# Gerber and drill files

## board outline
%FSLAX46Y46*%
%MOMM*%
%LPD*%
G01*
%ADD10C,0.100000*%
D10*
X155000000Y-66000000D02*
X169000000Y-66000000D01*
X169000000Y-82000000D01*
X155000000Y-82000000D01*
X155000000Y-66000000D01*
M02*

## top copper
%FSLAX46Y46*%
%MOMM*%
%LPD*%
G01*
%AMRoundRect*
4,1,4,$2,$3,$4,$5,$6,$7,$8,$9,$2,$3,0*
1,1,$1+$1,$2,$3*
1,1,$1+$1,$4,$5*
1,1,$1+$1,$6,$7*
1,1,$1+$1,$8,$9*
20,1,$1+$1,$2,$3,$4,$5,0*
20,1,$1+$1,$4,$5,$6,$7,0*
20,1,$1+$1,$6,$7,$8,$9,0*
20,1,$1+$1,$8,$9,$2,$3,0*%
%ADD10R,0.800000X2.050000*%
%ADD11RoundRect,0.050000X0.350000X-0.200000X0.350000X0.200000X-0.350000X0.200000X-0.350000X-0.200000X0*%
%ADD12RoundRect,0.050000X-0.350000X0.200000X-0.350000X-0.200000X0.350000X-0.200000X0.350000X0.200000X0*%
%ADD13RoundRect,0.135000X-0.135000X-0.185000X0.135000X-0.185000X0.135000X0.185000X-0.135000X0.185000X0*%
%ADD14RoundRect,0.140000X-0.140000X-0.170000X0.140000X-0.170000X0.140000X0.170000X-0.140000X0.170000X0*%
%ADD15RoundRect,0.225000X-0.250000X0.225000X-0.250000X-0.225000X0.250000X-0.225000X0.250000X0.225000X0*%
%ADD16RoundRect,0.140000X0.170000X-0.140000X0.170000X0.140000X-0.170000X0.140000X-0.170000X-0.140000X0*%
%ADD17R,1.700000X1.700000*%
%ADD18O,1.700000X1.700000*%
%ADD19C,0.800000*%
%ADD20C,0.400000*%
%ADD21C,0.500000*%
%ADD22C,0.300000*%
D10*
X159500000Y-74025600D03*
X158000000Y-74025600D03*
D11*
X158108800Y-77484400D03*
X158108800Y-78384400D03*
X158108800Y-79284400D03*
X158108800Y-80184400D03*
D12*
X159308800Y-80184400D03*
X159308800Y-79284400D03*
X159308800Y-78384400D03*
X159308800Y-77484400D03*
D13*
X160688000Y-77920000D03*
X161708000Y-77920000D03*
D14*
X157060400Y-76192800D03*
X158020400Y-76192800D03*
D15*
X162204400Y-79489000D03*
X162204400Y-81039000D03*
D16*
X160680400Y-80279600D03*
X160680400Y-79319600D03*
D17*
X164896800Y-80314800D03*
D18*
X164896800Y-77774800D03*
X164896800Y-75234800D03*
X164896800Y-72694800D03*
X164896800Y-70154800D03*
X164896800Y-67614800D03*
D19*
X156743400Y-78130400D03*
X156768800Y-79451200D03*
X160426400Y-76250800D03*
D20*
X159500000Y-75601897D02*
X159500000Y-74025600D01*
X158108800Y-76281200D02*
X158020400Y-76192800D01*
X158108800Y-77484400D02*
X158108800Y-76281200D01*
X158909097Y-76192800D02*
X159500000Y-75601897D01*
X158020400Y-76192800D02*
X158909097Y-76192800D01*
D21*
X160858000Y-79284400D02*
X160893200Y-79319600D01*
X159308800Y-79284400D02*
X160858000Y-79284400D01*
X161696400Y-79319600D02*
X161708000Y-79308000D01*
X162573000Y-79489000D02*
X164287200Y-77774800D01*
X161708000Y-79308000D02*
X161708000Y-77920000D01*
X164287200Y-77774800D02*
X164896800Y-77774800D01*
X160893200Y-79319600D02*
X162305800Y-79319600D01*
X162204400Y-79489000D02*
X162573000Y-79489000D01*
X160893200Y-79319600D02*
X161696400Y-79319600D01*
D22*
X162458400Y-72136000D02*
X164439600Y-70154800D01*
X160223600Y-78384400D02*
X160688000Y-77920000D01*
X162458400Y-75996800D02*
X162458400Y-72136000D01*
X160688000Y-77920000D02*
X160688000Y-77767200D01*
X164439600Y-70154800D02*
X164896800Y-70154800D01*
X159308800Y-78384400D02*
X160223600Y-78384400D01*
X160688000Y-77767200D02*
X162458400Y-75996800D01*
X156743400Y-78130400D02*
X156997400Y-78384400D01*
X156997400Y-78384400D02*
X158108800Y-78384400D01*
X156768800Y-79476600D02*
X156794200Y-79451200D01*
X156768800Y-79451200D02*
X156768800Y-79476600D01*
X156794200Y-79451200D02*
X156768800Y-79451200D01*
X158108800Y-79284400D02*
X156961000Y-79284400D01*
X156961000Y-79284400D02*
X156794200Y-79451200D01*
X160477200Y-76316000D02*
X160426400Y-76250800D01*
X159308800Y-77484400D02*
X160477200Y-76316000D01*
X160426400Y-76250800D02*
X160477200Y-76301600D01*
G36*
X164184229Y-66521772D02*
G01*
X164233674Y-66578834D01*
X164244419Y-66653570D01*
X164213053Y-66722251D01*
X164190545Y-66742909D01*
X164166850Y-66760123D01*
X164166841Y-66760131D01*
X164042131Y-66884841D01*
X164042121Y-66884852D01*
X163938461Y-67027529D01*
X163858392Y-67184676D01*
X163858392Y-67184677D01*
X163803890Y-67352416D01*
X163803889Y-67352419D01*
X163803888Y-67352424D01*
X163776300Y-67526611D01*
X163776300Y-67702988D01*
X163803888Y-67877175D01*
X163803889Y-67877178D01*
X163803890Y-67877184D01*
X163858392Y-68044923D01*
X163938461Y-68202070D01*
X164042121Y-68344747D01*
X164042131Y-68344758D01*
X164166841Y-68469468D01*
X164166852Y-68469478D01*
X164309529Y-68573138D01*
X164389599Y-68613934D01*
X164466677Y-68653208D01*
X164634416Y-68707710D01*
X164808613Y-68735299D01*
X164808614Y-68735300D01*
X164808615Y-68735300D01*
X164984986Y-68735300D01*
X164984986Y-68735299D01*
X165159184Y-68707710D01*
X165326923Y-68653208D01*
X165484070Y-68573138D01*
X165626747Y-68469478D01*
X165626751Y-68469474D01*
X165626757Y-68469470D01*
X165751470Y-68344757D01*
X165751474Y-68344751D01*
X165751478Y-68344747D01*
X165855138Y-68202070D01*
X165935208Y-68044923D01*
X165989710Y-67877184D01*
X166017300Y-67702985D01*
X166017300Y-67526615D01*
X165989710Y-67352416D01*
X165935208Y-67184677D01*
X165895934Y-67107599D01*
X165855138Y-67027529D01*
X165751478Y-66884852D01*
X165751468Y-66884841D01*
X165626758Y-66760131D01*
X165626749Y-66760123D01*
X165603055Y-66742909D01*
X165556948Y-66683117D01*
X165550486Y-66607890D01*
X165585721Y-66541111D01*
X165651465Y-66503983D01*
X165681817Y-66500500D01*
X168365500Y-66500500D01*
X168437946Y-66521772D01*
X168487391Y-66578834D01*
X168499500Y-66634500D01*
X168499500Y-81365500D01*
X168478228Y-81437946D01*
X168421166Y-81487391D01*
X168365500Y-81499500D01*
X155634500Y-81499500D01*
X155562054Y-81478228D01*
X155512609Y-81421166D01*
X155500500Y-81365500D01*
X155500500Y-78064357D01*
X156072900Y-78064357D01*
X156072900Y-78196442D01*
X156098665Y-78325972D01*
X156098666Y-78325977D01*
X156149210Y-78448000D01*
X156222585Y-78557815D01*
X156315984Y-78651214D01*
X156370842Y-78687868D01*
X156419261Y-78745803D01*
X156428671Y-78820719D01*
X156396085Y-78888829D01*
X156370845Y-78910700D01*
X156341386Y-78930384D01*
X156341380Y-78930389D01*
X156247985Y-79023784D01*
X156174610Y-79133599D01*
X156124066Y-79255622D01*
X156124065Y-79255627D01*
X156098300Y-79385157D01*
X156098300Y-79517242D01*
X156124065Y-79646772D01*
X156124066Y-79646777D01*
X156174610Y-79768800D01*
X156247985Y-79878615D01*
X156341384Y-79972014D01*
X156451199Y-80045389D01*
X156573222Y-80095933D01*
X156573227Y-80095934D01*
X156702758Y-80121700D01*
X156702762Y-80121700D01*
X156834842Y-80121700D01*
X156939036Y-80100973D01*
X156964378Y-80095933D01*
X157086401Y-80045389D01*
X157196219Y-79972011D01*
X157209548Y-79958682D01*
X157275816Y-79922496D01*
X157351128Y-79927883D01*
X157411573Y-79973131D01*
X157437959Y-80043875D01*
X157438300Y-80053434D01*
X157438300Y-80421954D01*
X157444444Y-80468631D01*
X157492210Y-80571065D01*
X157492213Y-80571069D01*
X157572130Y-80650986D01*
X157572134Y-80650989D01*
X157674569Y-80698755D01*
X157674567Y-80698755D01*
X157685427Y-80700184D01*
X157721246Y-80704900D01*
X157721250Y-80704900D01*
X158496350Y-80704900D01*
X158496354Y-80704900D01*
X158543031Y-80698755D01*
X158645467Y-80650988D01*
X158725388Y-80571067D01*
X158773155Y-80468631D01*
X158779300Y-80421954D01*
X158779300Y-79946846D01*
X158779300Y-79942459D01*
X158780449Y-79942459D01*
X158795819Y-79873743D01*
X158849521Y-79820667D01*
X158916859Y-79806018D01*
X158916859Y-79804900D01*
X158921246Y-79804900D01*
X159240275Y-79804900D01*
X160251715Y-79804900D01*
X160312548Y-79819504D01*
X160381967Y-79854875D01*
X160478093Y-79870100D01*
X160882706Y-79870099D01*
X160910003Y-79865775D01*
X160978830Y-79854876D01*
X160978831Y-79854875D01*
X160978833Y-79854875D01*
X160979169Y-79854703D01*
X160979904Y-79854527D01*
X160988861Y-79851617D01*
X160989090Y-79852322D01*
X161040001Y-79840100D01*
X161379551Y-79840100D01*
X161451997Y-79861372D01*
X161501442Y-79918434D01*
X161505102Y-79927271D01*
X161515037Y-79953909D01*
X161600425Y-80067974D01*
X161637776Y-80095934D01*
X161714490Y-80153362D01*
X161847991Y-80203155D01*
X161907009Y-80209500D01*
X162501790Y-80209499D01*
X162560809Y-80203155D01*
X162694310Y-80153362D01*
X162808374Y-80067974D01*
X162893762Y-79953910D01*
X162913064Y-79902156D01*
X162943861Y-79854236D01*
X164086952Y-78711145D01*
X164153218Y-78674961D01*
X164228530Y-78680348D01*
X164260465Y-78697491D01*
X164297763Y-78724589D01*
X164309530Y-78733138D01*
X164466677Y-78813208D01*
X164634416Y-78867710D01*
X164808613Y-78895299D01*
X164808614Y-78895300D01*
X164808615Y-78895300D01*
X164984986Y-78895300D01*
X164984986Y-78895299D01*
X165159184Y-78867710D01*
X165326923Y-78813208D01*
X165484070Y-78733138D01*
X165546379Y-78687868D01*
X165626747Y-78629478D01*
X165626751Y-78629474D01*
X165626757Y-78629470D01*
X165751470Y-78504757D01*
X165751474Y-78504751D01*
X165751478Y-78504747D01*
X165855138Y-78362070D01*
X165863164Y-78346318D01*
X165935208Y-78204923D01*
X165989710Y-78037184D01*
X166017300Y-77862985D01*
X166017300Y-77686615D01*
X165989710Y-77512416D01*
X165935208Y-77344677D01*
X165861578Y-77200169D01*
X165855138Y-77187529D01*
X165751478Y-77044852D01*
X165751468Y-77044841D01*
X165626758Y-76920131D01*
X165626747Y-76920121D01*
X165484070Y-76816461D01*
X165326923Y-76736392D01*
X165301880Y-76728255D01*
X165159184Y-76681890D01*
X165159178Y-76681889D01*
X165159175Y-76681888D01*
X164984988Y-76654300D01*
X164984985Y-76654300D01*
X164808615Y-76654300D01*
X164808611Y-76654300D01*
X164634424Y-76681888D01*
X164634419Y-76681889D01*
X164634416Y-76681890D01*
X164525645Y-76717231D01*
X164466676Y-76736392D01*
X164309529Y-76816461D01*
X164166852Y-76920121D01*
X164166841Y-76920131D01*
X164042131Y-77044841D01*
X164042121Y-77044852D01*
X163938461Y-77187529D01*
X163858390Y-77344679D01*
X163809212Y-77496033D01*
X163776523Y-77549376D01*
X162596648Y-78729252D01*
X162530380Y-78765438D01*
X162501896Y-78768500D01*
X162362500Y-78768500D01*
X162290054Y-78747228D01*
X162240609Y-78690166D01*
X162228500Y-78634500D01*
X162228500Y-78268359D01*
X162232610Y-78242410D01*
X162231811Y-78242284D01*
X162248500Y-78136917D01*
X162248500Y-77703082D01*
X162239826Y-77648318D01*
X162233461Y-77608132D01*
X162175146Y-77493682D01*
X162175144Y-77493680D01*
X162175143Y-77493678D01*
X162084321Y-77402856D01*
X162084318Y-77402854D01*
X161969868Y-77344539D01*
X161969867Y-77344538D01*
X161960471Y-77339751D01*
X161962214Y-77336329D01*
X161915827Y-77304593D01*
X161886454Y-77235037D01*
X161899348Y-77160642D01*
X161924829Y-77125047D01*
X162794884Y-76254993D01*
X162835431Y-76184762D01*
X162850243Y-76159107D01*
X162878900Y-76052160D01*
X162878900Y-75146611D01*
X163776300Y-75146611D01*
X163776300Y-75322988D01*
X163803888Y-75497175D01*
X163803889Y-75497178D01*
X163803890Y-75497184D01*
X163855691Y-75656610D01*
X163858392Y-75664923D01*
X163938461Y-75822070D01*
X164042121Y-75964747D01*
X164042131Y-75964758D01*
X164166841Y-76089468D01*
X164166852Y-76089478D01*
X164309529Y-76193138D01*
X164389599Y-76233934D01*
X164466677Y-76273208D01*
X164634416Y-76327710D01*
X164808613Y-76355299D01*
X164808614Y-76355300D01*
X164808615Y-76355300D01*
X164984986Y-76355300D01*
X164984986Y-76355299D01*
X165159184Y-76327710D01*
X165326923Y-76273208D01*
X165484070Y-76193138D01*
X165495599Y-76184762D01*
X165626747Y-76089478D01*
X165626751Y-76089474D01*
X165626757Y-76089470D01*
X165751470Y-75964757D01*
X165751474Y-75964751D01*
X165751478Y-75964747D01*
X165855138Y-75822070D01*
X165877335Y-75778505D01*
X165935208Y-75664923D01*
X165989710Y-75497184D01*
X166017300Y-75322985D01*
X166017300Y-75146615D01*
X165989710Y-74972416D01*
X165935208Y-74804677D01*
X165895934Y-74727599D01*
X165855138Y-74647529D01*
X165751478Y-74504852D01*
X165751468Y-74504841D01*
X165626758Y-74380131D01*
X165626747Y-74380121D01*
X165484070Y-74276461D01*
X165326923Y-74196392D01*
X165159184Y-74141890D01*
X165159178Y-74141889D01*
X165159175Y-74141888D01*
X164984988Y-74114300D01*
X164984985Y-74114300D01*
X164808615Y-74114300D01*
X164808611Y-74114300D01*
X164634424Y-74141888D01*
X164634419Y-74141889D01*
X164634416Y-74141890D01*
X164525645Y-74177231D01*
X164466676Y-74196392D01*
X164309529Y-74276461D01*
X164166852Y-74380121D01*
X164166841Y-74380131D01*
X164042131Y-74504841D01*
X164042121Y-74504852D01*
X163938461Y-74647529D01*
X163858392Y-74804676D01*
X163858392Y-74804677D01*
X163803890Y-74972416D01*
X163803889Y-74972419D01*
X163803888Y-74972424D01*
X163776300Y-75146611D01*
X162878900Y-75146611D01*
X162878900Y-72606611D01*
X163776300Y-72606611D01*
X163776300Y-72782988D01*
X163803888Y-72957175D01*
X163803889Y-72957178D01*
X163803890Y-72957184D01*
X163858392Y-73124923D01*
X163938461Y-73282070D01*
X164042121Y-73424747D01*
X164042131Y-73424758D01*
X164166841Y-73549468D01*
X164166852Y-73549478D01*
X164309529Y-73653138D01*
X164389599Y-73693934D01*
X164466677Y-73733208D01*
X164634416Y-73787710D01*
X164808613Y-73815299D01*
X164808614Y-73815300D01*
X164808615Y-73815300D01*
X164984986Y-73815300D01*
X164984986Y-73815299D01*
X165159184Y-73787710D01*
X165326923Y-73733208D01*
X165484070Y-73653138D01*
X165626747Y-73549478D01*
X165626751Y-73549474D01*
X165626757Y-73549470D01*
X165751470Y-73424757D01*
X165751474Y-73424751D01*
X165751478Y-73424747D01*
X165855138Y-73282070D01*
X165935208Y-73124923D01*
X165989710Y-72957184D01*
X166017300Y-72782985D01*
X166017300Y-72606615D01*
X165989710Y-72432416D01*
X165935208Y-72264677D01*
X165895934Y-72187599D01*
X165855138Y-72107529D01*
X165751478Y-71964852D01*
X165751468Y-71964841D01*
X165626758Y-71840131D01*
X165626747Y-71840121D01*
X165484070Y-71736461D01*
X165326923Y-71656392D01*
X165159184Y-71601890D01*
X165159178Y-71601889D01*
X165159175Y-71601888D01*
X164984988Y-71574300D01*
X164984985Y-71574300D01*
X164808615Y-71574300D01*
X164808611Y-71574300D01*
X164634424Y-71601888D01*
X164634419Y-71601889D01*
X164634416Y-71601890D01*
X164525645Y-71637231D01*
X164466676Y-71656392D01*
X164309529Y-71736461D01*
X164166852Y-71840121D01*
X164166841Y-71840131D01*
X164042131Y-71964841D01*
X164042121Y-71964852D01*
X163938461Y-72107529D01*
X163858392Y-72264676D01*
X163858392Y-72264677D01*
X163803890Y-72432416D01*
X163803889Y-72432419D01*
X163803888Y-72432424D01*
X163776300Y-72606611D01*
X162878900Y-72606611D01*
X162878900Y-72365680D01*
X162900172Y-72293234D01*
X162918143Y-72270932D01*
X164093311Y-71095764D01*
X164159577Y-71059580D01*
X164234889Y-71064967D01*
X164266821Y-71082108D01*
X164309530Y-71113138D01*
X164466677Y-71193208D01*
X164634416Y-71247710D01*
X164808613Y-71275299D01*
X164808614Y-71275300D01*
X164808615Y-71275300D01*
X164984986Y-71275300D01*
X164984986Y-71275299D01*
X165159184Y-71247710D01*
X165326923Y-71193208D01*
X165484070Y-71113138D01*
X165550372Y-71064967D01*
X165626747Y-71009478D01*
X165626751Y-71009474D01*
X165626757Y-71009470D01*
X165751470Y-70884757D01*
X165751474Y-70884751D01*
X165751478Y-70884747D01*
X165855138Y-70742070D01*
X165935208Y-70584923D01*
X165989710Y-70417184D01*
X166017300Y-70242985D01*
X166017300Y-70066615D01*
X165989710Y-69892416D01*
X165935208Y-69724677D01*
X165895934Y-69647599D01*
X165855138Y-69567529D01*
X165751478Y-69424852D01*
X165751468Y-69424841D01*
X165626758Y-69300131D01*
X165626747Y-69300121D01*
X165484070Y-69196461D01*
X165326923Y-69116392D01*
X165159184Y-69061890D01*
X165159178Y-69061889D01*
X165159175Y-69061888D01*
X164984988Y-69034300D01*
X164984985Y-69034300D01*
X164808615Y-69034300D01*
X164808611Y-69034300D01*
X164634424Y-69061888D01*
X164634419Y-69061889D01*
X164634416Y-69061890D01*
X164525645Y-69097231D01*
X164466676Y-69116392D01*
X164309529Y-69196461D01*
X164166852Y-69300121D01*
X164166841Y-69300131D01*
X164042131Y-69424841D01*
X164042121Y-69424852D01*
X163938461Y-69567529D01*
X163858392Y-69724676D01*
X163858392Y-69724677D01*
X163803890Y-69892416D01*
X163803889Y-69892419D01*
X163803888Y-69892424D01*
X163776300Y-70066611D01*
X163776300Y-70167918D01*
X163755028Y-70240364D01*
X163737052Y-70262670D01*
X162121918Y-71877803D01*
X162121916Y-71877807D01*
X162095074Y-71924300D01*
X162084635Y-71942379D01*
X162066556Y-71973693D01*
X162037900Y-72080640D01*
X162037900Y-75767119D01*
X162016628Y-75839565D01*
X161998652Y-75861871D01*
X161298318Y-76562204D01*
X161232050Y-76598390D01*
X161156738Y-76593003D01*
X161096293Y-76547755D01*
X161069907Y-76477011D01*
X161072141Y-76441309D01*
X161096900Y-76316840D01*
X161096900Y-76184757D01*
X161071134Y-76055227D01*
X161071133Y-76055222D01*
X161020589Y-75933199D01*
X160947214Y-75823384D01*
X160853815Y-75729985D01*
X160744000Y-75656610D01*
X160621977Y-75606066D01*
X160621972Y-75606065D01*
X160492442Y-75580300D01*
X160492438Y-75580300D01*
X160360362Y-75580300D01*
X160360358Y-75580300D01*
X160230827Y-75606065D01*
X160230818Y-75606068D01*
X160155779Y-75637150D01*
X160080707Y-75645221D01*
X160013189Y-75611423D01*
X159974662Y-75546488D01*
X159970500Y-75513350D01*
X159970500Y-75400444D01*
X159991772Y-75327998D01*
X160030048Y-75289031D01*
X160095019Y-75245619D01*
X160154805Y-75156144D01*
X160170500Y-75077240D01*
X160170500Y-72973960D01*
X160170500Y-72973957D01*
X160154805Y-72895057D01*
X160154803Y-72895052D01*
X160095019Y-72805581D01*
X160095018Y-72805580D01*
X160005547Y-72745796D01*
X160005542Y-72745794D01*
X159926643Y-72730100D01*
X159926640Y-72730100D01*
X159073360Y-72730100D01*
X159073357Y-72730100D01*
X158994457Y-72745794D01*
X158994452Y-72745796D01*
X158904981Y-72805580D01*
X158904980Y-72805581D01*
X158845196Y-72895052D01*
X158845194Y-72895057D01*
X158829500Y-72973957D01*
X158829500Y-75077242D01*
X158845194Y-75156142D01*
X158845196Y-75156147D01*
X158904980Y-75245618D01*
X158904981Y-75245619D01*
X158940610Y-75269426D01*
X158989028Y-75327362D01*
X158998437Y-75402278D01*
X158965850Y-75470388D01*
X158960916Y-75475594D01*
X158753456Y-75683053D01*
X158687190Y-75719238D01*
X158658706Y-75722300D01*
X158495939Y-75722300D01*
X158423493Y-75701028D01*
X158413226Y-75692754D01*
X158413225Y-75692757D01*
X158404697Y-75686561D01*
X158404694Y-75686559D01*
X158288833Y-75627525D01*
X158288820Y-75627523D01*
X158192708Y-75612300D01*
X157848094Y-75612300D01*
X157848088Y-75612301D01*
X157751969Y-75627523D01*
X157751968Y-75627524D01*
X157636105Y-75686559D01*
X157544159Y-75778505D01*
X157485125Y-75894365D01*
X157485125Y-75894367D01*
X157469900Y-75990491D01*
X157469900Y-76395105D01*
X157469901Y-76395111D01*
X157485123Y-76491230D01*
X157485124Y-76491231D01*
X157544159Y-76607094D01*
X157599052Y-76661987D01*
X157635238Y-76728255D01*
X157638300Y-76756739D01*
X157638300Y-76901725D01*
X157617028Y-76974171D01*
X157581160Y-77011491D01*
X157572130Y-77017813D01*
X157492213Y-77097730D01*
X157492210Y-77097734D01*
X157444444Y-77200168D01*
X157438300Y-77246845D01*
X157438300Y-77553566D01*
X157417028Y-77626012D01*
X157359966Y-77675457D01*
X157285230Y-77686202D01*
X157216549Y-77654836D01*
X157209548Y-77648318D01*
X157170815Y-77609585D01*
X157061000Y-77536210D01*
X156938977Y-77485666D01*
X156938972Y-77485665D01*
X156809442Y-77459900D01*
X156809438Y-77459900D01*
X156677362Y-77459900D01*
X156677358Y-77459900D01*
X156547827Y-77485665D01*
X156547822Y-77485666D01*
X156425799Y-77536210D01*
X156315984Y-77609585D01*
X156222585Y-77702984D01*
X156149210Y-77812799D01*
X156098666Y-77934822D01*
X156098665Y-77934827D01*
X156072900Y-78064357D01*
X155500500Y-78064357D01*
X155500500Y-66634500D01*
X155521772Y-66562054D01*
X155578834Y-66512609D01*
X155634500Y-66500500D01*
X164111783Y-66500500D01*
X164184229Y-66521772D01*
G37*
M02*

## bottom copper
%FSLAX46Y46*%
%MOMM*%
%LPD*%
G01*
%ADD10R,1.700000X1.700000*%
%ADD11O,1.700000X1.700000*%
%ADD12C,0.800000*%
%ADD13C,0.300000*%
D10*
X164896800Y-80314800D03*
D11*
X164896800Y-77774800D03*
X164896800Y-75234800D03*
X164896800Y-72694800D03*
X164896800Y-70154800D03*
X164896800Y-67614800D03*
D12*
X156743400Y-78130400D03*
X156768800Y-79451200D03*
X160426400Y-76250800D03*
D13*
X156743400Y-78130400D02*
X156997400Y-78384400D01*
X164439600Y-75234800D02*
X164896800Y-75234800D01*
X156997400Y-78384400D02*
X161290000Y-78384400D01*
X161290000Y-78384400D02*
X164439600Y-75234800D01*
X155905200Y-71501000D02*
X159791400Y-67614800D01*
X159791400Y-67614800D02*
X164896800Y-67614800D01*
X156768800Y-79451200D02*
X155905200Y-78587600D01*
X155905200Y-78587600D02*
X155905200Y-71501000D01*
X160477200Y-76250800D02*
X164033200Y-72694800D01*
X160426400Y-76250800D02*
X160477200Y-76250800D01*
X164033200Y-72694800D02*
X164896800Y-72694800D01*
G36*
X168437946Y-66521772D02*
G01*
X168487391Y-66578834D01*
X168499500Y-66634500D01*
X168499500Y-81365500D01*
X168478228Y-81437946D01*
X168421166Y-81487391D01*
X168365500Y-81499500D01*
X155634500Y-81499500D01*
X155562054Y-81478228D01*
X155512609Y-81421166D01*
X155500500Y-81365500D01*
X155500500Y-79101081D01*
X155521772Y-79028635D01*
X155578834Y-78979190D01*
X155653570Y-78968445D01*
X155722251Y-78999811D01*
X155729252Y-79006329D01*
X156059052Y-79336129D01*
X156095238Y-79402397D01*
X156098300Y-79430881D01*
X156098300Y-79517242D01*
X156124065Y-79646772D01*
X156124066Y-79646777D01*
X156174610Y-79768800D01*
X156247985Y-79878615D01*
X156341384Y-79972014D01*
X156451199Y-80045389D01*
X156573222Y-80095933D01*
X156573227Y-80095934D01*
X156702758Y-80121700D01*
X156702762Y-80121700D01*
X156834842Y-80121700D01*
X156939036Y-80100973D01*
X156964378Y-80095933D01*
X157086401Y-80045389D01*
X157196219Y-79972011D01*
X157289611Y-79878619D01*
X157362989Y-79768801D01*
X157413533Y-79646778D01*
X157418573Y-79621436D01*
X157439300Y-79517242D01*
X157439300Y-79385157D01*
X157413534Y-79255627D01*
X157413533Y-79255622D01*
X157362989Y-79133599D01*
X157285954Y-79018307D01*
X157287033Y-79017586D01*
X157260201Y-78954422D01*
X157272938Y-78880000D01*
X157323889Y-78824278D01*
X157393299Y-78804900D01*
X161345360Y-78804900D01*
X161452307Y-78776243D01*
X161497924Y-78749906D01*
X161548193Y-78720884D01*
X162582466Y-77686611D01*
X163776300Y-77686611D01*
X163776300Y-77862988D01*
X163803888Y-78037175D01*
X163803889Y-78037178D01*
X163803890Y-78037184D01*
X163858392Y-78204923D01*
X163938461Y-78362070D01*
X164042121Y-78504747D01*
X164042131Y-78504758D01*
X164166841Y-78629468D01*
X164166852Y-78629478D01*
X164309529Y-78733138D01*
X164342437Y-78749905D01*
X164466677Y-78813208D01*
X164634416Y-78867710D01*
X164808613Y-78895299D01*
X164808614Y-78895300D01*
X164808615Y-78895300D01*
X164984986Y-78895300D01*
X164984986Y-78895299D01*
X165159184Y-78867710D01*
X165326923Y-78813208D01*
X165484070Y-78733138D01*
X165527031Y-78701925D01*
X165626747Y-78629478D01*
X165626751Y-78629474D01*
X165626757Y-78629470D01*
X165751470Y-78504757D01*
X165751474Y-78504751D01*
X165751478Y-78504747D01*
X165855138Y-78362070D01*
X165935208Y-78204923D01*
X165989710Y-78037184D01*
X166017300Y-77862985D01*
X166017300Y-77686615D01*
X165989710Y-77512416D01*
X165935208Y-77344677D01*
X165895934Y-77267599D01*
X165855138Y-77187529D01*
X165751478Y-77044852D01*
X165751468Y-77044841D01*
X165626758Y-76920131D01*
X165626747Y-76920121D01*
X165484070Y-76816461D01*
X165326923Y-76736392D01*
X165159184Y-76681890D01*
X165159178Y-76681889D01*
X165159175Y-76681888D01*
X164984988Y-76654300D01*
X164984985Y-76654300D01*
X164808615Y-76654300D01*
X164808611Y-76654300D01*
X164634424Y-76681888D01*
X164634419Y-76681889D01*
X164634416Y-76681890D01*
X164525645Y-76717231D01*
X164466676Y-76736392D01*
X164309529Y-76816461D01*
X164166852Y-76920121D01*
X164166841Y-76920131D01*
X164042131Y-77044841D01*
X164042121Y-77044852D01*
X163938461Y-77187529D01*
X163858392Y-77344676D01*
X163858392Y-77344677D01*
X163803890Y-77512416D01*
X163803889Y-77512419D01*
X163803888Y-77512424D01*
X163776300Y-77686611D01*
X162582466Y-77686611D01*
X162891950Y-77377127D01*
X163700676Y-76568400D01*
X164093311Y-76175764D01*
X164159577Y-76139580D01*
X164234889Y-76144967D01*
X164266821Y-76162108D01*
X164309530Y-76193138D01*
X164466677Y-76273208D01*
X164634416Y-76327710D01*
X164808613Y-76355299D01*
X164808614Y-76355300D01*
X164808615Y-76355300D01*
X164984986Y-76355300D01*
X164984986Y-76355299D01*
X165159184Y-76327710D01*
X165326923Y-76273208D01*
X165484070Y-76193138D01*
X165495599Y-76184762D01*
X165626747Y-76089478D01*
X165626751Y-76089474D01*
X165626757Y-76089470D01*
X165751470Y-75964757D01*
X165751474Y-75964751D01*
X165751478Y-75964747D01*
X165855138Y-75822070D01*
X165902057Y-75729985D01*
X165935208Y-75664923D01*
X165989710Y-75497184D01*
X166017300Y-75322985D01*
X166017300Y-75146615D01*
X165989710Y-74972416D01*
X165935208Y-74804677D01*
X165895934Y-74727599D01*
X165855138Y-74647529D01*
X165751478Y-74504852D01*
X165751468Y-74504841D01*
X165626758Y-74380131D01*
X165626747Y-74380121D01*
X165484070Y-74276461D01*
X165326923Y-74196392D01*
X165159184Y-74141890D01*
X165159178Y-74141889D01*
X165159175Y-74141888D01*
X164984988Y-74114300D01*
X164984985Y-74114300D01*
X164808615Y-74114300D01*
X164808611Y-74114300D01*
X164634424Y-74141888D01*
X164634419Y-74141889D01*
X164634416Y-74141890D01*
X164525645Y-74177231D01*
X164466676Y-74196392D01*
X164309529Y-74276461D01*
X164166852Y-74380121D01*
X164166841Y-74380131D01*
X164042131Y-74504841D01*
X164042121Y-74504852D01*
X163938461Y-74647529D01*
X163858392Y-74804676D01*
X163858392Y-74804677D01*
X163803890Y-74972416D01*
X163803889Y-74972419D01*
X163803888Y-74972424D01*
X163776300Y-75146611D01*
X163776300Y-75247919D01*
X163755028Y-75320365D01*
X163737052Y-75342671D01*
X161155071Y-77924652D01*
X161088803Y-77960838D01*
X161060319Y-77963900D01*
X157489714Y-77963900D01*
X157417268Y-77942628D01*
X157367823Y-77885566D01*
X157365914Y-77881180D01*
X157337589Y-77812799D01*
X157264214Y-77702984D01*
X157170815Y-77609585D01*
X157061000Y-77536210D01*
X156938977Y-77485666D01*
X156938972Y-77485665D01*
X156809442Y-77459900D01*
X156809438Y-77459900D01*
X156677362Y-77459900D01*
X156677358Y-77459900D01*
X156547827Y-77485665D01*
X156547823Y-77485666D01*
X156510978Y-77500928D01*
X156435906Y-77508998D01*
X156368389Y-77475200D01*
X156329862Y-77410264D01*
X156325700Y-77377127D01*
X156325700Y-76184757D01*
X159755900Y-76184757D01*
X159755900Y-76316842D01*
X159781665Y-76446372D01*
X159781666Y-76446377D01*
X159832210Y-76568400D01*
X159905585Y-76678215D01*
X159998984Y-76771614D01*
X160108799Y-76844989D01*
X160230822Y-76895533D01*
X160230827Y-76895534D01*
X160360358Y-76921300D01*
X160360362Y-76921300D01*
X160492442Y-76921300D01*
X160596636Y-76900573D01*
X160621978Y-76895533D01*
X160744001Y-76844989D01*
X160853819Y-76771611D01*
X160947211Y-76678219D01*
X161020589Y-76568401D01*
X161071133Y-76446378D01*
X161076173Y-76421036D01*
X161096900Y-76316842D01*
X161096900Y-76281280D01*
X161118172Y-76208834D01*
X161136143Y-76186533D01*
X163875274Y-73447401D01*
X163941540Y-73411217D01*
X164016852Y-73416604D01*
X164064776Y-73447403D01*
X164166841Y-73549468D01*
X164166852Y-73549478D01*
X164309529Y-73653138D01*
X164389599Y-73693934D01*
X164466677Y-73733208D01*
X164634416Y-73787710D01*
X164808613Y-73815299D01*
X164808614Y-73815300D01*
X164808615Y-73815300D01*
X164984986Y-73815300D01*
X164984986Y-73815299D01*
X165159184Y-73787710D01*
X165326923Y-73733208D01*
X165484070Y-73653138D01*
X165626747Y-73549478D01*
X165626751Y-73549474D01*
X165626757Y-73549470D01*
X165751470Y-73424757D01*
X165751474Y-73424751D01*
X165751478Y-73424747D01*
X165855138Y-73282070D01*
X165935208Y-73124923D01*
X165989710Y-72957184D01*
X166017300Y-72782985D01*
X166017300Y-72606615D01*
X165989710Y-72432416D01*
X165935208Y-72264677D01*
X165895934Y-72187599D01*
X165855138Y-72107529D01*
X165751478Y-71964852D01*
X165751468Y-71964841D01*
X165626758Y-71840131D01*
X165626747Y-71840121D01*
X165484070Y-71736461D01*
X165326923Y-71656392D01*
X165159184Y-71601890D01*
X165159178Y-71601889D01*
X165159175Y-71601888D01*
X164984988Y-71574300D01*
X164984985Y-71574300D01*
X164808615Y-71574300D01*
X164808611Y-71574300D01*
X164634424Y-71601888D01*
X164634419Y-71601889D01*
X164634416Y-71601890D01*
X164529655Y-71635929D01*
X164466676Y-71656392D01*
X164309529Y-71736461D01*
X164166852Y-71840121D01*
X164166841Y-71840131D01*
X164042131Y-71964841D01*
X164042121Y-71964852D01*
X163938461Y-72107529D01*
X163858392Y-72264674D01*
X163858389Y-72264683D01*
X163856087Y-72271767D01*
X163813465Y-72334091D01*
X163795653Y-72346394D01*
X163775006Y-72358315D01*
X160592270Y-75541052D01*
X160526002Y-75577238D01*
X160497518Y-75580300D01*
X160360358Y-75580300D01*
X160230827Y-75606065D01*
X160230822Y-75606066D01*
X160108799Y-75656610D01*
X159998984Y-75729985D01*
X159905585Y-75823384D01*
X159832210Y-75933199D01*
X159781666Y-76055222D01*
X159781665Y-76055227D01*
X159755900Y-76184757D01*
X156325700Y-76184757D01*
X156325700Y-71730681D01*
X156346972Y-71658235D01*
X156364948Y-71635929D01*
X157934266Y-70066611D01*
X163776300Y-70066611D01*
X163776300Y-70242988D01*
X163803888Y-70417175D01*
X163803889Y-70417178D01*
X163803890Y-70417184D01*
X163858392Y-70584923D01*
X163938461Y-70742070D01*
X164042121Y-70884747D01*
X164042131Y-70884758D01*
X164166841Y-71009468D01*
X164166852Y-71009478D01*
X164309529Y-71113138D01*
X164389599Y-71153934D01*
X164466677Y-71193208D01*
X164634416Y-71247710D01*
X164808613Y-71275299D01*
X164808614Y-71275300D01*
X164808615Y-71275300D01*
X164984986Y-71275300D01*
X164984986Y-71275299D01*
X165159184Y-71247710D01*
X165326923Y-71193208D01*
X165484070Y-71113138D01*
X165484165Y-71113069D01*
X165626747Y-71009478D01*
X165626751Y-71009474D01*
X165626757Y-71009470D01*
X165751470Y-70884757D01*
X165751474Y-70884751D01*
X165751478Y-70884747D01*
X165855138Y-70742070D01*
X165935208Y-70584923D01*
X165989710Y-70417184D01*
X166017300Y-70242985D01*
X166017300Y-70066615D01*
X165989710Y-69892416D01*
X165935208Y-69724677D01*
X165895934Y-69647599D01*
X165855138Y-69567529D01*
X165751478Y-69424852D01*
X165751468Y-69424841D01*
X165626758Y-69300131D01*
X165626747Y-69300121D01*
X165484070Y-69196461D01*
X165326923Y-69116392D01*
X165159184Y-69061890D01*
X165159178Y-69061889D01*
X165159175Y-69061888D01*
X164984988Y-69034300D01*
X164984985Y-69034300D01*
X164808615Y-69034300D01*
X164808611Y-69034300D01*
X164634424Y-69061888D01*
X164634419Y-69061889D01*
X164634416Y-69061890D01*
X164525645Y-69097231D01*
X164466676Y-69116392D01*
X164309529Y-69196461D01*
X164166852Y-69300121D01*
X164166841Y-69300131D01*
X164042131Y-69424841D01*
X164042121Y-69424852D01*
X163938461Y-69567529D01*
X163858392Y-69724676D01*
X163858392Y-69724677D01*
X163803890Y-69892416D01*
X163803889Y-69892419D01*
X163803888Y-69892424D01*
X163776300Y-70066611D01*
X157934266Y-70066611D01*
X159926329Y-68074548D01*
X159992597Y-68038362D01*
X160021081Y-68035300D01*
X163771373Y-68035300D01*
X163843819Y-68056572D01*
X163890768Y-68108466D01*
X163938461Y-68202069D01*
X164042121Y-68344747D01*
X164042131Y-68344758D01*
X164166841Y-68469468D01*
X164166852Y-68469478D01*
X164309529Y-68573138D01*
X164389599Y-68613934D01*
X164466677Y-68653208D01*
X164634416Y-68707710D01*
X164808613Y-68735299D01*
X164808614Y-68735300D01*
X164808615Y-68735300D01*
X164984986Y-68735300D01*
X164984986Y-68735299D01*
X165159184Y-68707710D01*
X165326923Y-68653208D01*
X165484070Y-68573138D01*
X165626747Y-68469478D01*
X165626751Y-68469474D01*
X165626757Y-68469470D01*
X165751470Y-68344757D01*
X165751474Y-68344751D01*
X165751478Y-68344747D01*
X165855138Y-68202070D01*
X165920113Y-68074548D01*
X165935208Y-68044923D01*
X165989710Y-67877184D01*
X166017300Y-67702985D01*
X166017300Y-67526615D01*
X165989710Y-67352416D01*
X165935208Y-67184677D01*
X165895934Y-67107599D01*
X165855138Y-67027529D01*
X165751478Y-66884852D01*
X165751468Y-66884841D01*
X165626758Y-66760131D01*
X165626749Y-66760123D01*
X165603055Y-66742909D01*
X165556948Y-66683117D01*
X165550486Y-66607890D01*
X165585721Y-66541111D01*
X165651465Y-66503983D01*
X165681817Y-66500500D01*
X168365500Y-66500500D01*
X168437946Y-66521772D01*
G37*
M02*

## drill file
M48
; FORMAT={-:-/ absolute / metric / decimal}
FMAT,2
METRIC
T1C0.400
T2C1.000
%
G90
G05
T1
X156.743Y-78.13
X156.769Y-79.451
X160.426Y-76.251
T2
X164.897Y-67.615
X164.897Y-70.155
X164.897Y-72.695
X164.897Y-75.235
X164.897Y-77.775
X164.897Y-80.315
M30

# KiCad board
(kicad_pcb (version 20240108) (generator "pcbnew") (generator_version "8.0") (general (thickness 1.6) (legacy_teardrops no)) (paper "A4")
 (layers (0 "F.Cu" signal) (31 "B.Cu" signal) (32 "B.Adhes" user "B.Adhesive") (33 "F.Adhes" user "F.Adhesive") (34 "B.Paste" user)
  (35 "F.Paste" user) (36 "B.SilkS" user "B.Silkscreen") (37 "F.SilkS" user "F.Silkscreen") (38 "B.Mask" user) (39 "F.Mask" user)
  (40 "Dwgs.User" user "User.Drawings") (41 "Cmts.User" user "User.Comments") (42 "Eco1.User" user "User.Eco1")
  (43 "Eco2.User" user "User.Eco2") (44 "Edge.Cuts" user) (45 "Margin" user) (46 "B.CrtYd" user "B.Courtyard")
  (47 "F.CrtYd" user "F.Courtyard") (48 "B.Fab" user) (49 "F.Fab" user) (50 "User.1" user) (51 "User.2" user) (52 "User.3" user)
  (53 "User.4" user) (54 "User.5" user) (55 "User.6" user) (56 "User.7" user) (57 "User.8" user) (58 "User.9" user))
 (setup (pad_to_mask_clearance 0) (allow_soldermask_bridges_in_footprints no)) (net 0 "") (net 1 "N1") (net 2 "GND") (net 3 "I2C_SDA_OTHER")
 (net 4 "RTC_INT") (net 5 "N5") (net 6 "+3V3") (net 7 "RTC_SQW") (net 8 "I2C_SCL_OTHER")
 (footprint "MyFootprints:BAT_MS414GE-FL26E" (layer "F.Cu") (at 158.75 70.3006 -90)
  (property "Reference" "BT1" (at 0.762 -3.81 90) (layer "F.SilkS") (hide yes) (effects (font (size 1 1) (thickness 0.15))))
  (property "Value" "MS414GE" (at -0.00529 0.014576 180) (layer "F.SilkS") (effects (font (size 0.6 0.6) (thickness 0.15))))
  (pad "1" smd rect (at 3.725 -0.75 270) (size 2.05 0.8) (layers "F.Cu" "F.Paste" "F.Mask") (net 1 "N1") (solder_mask_margin 0.102))
  (pad "2" smd rect (at 3.725 0.75 270) (size 2.05 0.8) (layers "F.Cu" "F.Paste" "F.Mask") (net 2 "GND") (solder_mask_margin 0.102)))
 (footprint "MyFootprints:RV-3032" (layer "F.Cu") (at 158.7088 78.8344 -90)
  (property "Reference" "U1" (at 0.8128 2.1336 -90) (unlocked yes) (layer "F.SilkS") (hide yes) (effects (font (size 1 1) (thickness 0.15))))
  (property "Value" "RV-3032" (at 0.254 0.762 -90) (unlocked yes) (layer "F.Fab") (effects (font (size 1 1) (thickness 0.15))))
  (pad "1" smd roundrect (at -1.35 0.6 90) (size 0.5 0.8) (layers "F.Cu" "F.Paste" "F.Mask") (roundrect_rratio 0.1) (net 1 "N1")
   (thermal_bridge_angle 45))
  (pad "2" smd roundrect (at -0.45 0.6 90) (size 0.5 0.8) (layers "F.Cu" "F.Paste" "F.Mask") (roundrect_rratio 0.1) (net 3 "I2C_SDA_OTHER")
   (thermal_bridge_angle 45))
  (pad "3" smd roundrect (at 0.45 0.6 90) (size 0.5 0.8) (layers "F.Cu" "F.Paste" "F.Mask") (roundrect_rratio 0.1) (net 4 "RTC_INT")
   (thermal_bridge_angle 45))
  (pad "4" smd roundrect (at 1.35 0.6 90) (size 0.5 0.8) (layers "F.Cu" "F.Paste" "F.Mask") (roundrect_rratio 0.1) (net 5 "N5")
   (thermal_bridge_angle 45))
  (pad "5" smd roundrect (at 1.35 -0.6 270) (size 0.5 0.8) (layers "F.Cu" "F.Paste" "F.Mask") (roundrect_rratio 0.1) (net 2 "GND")
   (thermal_bridge_angle 45))
  (pad "6" smd roundrect (at 0.45 -0.6 270) (size 0.5 0.8) (layers "F.Cu" "F.Paste" "F.Mask") (roundrect_rratio 0.1) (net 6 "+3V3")
   (thermal_bridge_angle 45))
  (pad "7" smd roundrect (at -0.45 -0.6 270) (size 0.5 0.8) (layers "F.Cu" "F.Paste" "F.Mask") (roundrect_rratio 0.1) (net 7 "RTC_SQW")
   (thermal_bridge_angle 45))
  (pad "8" smd roundrect (at -1.35 -0.6 270) (size 0.5 0.8) (layers "F.Cu" "F.Paste" "F.Mask") (roundrect_rratio 0.1)
   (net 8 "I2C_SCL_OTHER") (thermal_bridge_angle 45)))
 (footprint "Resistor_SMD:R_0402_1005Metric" (layer "F.Cu") (at 161.198 77.92)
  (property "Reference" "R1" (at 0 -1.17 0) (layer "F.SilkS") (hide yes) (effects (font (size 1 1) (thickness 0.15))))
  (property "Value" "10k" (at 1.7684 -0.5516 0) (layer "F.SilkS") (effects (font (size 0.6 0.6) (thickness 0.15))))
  (pad "1" smd roundrect (at -0.51 0) (size 0.54 0.64) (layers "F.Cu" "F.Paste" "F.Mask") (roundrect_rratio 0.25) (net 7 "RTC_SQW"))
  (pad "2" smd roundrect (at 0.51 0) (size 0.54 0.64) (layers "F.Cu" "F.Paste" "F.Mask") (roundrect_rratio 0.25) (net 6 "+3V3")))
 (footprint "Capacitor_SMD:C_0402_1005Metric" (layer "F.Cu") (at 157.5404 76.1928)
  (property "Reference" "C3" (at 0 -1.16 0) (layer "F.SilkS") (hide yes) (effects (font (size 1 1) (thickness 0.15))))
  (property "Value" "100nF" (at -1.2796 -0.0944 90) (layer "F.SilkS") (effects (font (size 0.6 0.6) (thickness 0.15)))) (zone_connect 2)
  (pad "1" smd roundrect (at -0.48 0) (size 0.56 0.62) (layers "F.Cu" "F.Paste" "F.Mask") (roundrect_rratio 0.25) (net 2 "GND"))
  (pad "2" smd roundrect (at 0.48 0) (size 0.56 0.62) (layers "F.Cu" "F.Paste" "F.Mask") (roundrect_rratio 0.25) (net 1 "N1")))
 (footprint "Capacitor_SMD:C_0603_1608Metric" (layer "F.Cu") (at 162.2044 80.264 -90)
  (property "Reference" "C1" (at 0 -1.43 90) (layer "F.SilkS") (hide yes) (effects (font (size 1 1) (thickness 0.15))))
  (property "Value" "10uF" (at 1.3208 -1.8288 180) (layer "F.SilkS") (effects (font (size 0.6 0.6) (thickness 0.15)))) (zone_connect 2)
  (pad "1" smd roundrect (at -0.775 0 270) (size 0.9 0.95) (layers "F.Cu" "F.Paste" "F.Mask") (roundrect_rratio 0.25) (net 6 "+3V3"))
  (pad "2" smd roundrect (at 0.775 0 270) (size 0.9 0.95) (layers "F.Cu" "F.Paste" "F.Mask") (roundrect_rratio 0.25) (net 2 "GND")))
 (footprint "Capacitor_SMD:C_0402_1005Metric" (layer "F.Cu") (at 160.6804 79.7996 90)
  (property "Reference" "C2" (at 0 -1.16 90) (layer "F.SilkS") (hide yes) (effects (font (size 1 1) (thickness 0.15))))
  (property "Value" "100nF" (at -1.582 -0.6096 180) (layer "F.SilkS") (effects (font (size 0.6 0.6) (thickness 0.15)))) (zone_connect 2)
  (pad "1" smd roundrect (at -0.48 0 90) (size 0.56 0.62) (layers "F.Cu" "F.Paste" "F.Mask") (roundrect_rratio 0.25) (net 2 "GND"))
  (pad "2" smd roundrect (at 0.48 0 90) (size 0.56 0.62) (layers "F.Cu" "F.Paste" "F.Mask") (roundrect_rratio 0.25) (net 6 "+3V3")))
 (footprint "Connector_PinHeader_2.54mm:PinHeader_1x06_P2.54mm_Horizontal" (layer "B.Cu") (at 164.8968 80.3148)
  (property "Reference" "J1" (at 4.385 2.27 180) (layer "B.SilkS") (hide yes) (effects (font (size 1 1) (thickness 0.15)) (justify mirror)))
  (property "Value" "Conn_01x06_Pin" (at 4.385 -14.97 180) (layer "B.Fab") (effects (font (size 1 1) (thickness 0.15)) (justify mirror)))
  (pad "1" thru_hole rect (at 0 0) (size 1.7 1.7) (drill 1) (layers "*.Cu" "*.Mask") (remove_unused_layers no) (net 2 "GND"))
  (pad "2" thru_hole oval (at 0 -2.54) (size 1.7 1.7) (drill 1) (layers "*.Cu" "*.Mask") (remove_unused_layers no) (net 6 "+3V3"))
  (pad "3" thru_hole oval (at 0 -5.08) (size 1.7 1.7) (drill 1) (layers "*.Cu" "*.Mask") (remove_unused_layers no) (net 3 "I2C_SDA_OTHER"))
  (pad "4" thru_hole oval (at 0 -7.62) (size 1.7 1.7) (drill 1) (layers "*.Cu" "*.Mask") (remove_unused_layers no) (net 8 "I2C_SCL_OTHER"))
  (pad "5" thru_hole oval (at 0 -10.16) (size 1.7 1.7) (drill 1) (layers "*.Cu" "*.Mask") (remove_unused_layers no) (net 7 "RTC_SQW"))
  (pad "6" thru_hole oval (at 0 -12.7) (size 1.7 1.7) (drill 1) (layers "*.Cu" "*.Mask") (remove_unused_layers no) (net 4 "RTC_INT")))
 (gr_rect (start 155 66) (end 169 82) (stroke (width 0.1) (type default)) (fill none) (layer "Edge.Cuts"))
 (segment (start 159.5 75.601897) (end 159.5 74.0256) (width 0.4) (layer "F.Cu") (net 1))
 (segment (start 158.1088 76.2812) (end 158.0204 76.1928) (width 0.4) (layer "F.Cu") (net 1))
 (segment (start 158.1088 77.4844) (end 158.1088 76.2812) (width 0.4) (layer "F.Cu") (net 1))
 (segment (start 158.909097 76.1928) (end 159.5 75.601897) (width 0.4) (layer "F.Cu") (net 1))
 (segment (start 158.0204 76.1928) (end 158.909097 76.1928) (width 0.4) (layer "F.Cu") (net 1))
 (segment (start 160.858 79.2844) (end 160.8932 79.3196) (width 0.5) (layer "F.Cu") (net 6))
 (segment (start 159.3088 79.2844) (end 160.858 79.2844) (width 0.5) (layer "F.Cu") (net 6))
 (segment (start 161.6964 79.3196) (end 161.708 79.308) (width 0.5) (layer "F.Cu") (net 6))
 (segment (start 162.573 79.489) (end 164.2872 77.7748) (width 0.5) (layer "F.Cu") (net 6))
 (segment (start 161.708 79.308) (end 161.708 77.92) (width 0.5) (layer "F.Cu") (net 6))
 (segment (start 164.2872 77.7748) (end 164.8968 77.7748) (width 0.5) (layer "F.Cu") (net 6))
 (segment (start 160.8932 79.3196) (end 162.3058 79.3196) (width 0.5) (layer "F.Cu") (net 6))
 (segment (start 162.2044 79.489) (end 162.573 79.489) (width 0.5) (layer "F.Cu") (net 6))
 (segment (start 160.8932 79.3196) (end 161.6964 79.3196) (width 0.5) (layer "F.Cu") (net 6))
 (segment (start 162.4584 72.136) (end 164.4396 70.1548) (width 0.3) (layer "F.Cu") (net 7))
 (segment (start 160.2236 78.3844) (end 160.688 77.92) (width 0.3) (layer "F.Cu") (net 7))
 (segment (start 162.4584 75.9968) (end 162.4584 72.136) (width 0.3) (layer "F.Cu") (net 7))
 (segment (start 160.688 77.92) (end 160.688 77.7672) (width 0.3) (layer "F.Cu") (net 7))
 (segment (start 164.4396 70.1548) (end 164.8968 70.1548) (width 0.3) (layer "F.Cu") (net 7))
 (segment (start 159.3088 78.3844) (end 160.2236 78.3844) (width 0.3) (layer "F.Cu") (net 7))
 (segment (start 160.688 77.7672) (end 162.4584 75.9968) (width 0.3) (layer "F.Cu") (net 7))
 (segment (start 156.7434 78.1304) (end 156.9974 78.3844) (width 0.3) (layer "F.Cu") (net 3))
 (segment (start 156.9974 78.3844) (end 158.1088 78.3844) (width 0.3) (layer "F.Cu") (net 3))
 (via (at 156.7434 78.1304) (size 0.8) (drill 0.4) (layers "F.Cu" "B.Cu") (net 3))
 (segment (start 156.7434 78.1304) (end 156.9974 78.3844) (width 0.3) (layer "B.Cu") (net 3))
 (segment (start 164.4396 75.2348) (end 164.8968 75.2348) (width 0.3) (layer "B.Cu") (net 3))
 (segment (start 156.9974 78.3844) (end 161.29 78.3844) (width 0.3) (layer "B.Cu") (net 3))
 (segment (start 161.29 78.3844) (end 164.4396 75.2348) (width 0.3) (layer "B.Cu") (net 3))
 (segment (start 156.7688 79.4766) (end 156.7942 79.4512) (width 0.3) (layer "F.Cu") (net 4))
 (segment (start 156.7688 79.4512) (end 156.7688 79.4766) (width 0.3) (layer "F.Cu") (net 4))
 (segment (start 156.7942 79.4512) (end 156.7688 79.4512) (width 0.3) (layer "F.Cu") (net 4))
 (segment (start 158.1088 79.2844) (end 156.961 79.2844) (width 0.3) (layer "F.Cu") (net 4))
 (segment (start 156.961 79.2844) (end 156.7942 79.4512) (width 0.3) (layer "F.Cu") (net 4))
 (via (at 156.7688 79.4512) (size 0.8) (drill 0.4) (layers "F.Cu" "B.Cu") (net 4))
 (segment (start 155.9052 71.501) (end 159.7914 67.6148) (width 0.3) (layer "B.Cu") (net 4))
 (segment (start 159.7914 67.6148) (end 164.8968 67.6148) (width 0.3) (layer "B.Cu") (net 4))
 (segment (start 156.7688 79.4512) (end 155.9052 78.5876) (width 0.3) (layer "B.Cu") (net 4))
 (segment (start 155.9052 78.5876) (end 155.9052 71.501) (width 0.3) (layer "B.Cu") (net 4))
 (segment (start 160.4772 76.316) (end 160.4264 76.2508) (width 0.3) (layer "F.Cu") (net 8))
 (segment (start 159.3088 77.4844) (end 160.4772 76.316) (width 0.3) (layer "F.Cu") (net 8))
 (segment (start 160.4264 76.2508) (end 160.4772 76.3016) (width 0.3) (layer "F.Cu") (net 8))
 (via (at 160.4264 76.2508) (size 0.8) (drill 0.4) (layers "F.Cu" "B.Cu") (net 8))
 (segment (start 160.4772 76.2508) (end 164.0332 72.6948) (width 0.3) (layer "B.Cu") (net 8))
 (segment (start 160.4264 76.2508) (end 160.4772 76.2508) (width 0.3) (layer "B.Cu") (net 8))
 (segment (start 164.0332 72.6948) (end 164.8968 72.6948) (width 0.3) (layer "B.Cu") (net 8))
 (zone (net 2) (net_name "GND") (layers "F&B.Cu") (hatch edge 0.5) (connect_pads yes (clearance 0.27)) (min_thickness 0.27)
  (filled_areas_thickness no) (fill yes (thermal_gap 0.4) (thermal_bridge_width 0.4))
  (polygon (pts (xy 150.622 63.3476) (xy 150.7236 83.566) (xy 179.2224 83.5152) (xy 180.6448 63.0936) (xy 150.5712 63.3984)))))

